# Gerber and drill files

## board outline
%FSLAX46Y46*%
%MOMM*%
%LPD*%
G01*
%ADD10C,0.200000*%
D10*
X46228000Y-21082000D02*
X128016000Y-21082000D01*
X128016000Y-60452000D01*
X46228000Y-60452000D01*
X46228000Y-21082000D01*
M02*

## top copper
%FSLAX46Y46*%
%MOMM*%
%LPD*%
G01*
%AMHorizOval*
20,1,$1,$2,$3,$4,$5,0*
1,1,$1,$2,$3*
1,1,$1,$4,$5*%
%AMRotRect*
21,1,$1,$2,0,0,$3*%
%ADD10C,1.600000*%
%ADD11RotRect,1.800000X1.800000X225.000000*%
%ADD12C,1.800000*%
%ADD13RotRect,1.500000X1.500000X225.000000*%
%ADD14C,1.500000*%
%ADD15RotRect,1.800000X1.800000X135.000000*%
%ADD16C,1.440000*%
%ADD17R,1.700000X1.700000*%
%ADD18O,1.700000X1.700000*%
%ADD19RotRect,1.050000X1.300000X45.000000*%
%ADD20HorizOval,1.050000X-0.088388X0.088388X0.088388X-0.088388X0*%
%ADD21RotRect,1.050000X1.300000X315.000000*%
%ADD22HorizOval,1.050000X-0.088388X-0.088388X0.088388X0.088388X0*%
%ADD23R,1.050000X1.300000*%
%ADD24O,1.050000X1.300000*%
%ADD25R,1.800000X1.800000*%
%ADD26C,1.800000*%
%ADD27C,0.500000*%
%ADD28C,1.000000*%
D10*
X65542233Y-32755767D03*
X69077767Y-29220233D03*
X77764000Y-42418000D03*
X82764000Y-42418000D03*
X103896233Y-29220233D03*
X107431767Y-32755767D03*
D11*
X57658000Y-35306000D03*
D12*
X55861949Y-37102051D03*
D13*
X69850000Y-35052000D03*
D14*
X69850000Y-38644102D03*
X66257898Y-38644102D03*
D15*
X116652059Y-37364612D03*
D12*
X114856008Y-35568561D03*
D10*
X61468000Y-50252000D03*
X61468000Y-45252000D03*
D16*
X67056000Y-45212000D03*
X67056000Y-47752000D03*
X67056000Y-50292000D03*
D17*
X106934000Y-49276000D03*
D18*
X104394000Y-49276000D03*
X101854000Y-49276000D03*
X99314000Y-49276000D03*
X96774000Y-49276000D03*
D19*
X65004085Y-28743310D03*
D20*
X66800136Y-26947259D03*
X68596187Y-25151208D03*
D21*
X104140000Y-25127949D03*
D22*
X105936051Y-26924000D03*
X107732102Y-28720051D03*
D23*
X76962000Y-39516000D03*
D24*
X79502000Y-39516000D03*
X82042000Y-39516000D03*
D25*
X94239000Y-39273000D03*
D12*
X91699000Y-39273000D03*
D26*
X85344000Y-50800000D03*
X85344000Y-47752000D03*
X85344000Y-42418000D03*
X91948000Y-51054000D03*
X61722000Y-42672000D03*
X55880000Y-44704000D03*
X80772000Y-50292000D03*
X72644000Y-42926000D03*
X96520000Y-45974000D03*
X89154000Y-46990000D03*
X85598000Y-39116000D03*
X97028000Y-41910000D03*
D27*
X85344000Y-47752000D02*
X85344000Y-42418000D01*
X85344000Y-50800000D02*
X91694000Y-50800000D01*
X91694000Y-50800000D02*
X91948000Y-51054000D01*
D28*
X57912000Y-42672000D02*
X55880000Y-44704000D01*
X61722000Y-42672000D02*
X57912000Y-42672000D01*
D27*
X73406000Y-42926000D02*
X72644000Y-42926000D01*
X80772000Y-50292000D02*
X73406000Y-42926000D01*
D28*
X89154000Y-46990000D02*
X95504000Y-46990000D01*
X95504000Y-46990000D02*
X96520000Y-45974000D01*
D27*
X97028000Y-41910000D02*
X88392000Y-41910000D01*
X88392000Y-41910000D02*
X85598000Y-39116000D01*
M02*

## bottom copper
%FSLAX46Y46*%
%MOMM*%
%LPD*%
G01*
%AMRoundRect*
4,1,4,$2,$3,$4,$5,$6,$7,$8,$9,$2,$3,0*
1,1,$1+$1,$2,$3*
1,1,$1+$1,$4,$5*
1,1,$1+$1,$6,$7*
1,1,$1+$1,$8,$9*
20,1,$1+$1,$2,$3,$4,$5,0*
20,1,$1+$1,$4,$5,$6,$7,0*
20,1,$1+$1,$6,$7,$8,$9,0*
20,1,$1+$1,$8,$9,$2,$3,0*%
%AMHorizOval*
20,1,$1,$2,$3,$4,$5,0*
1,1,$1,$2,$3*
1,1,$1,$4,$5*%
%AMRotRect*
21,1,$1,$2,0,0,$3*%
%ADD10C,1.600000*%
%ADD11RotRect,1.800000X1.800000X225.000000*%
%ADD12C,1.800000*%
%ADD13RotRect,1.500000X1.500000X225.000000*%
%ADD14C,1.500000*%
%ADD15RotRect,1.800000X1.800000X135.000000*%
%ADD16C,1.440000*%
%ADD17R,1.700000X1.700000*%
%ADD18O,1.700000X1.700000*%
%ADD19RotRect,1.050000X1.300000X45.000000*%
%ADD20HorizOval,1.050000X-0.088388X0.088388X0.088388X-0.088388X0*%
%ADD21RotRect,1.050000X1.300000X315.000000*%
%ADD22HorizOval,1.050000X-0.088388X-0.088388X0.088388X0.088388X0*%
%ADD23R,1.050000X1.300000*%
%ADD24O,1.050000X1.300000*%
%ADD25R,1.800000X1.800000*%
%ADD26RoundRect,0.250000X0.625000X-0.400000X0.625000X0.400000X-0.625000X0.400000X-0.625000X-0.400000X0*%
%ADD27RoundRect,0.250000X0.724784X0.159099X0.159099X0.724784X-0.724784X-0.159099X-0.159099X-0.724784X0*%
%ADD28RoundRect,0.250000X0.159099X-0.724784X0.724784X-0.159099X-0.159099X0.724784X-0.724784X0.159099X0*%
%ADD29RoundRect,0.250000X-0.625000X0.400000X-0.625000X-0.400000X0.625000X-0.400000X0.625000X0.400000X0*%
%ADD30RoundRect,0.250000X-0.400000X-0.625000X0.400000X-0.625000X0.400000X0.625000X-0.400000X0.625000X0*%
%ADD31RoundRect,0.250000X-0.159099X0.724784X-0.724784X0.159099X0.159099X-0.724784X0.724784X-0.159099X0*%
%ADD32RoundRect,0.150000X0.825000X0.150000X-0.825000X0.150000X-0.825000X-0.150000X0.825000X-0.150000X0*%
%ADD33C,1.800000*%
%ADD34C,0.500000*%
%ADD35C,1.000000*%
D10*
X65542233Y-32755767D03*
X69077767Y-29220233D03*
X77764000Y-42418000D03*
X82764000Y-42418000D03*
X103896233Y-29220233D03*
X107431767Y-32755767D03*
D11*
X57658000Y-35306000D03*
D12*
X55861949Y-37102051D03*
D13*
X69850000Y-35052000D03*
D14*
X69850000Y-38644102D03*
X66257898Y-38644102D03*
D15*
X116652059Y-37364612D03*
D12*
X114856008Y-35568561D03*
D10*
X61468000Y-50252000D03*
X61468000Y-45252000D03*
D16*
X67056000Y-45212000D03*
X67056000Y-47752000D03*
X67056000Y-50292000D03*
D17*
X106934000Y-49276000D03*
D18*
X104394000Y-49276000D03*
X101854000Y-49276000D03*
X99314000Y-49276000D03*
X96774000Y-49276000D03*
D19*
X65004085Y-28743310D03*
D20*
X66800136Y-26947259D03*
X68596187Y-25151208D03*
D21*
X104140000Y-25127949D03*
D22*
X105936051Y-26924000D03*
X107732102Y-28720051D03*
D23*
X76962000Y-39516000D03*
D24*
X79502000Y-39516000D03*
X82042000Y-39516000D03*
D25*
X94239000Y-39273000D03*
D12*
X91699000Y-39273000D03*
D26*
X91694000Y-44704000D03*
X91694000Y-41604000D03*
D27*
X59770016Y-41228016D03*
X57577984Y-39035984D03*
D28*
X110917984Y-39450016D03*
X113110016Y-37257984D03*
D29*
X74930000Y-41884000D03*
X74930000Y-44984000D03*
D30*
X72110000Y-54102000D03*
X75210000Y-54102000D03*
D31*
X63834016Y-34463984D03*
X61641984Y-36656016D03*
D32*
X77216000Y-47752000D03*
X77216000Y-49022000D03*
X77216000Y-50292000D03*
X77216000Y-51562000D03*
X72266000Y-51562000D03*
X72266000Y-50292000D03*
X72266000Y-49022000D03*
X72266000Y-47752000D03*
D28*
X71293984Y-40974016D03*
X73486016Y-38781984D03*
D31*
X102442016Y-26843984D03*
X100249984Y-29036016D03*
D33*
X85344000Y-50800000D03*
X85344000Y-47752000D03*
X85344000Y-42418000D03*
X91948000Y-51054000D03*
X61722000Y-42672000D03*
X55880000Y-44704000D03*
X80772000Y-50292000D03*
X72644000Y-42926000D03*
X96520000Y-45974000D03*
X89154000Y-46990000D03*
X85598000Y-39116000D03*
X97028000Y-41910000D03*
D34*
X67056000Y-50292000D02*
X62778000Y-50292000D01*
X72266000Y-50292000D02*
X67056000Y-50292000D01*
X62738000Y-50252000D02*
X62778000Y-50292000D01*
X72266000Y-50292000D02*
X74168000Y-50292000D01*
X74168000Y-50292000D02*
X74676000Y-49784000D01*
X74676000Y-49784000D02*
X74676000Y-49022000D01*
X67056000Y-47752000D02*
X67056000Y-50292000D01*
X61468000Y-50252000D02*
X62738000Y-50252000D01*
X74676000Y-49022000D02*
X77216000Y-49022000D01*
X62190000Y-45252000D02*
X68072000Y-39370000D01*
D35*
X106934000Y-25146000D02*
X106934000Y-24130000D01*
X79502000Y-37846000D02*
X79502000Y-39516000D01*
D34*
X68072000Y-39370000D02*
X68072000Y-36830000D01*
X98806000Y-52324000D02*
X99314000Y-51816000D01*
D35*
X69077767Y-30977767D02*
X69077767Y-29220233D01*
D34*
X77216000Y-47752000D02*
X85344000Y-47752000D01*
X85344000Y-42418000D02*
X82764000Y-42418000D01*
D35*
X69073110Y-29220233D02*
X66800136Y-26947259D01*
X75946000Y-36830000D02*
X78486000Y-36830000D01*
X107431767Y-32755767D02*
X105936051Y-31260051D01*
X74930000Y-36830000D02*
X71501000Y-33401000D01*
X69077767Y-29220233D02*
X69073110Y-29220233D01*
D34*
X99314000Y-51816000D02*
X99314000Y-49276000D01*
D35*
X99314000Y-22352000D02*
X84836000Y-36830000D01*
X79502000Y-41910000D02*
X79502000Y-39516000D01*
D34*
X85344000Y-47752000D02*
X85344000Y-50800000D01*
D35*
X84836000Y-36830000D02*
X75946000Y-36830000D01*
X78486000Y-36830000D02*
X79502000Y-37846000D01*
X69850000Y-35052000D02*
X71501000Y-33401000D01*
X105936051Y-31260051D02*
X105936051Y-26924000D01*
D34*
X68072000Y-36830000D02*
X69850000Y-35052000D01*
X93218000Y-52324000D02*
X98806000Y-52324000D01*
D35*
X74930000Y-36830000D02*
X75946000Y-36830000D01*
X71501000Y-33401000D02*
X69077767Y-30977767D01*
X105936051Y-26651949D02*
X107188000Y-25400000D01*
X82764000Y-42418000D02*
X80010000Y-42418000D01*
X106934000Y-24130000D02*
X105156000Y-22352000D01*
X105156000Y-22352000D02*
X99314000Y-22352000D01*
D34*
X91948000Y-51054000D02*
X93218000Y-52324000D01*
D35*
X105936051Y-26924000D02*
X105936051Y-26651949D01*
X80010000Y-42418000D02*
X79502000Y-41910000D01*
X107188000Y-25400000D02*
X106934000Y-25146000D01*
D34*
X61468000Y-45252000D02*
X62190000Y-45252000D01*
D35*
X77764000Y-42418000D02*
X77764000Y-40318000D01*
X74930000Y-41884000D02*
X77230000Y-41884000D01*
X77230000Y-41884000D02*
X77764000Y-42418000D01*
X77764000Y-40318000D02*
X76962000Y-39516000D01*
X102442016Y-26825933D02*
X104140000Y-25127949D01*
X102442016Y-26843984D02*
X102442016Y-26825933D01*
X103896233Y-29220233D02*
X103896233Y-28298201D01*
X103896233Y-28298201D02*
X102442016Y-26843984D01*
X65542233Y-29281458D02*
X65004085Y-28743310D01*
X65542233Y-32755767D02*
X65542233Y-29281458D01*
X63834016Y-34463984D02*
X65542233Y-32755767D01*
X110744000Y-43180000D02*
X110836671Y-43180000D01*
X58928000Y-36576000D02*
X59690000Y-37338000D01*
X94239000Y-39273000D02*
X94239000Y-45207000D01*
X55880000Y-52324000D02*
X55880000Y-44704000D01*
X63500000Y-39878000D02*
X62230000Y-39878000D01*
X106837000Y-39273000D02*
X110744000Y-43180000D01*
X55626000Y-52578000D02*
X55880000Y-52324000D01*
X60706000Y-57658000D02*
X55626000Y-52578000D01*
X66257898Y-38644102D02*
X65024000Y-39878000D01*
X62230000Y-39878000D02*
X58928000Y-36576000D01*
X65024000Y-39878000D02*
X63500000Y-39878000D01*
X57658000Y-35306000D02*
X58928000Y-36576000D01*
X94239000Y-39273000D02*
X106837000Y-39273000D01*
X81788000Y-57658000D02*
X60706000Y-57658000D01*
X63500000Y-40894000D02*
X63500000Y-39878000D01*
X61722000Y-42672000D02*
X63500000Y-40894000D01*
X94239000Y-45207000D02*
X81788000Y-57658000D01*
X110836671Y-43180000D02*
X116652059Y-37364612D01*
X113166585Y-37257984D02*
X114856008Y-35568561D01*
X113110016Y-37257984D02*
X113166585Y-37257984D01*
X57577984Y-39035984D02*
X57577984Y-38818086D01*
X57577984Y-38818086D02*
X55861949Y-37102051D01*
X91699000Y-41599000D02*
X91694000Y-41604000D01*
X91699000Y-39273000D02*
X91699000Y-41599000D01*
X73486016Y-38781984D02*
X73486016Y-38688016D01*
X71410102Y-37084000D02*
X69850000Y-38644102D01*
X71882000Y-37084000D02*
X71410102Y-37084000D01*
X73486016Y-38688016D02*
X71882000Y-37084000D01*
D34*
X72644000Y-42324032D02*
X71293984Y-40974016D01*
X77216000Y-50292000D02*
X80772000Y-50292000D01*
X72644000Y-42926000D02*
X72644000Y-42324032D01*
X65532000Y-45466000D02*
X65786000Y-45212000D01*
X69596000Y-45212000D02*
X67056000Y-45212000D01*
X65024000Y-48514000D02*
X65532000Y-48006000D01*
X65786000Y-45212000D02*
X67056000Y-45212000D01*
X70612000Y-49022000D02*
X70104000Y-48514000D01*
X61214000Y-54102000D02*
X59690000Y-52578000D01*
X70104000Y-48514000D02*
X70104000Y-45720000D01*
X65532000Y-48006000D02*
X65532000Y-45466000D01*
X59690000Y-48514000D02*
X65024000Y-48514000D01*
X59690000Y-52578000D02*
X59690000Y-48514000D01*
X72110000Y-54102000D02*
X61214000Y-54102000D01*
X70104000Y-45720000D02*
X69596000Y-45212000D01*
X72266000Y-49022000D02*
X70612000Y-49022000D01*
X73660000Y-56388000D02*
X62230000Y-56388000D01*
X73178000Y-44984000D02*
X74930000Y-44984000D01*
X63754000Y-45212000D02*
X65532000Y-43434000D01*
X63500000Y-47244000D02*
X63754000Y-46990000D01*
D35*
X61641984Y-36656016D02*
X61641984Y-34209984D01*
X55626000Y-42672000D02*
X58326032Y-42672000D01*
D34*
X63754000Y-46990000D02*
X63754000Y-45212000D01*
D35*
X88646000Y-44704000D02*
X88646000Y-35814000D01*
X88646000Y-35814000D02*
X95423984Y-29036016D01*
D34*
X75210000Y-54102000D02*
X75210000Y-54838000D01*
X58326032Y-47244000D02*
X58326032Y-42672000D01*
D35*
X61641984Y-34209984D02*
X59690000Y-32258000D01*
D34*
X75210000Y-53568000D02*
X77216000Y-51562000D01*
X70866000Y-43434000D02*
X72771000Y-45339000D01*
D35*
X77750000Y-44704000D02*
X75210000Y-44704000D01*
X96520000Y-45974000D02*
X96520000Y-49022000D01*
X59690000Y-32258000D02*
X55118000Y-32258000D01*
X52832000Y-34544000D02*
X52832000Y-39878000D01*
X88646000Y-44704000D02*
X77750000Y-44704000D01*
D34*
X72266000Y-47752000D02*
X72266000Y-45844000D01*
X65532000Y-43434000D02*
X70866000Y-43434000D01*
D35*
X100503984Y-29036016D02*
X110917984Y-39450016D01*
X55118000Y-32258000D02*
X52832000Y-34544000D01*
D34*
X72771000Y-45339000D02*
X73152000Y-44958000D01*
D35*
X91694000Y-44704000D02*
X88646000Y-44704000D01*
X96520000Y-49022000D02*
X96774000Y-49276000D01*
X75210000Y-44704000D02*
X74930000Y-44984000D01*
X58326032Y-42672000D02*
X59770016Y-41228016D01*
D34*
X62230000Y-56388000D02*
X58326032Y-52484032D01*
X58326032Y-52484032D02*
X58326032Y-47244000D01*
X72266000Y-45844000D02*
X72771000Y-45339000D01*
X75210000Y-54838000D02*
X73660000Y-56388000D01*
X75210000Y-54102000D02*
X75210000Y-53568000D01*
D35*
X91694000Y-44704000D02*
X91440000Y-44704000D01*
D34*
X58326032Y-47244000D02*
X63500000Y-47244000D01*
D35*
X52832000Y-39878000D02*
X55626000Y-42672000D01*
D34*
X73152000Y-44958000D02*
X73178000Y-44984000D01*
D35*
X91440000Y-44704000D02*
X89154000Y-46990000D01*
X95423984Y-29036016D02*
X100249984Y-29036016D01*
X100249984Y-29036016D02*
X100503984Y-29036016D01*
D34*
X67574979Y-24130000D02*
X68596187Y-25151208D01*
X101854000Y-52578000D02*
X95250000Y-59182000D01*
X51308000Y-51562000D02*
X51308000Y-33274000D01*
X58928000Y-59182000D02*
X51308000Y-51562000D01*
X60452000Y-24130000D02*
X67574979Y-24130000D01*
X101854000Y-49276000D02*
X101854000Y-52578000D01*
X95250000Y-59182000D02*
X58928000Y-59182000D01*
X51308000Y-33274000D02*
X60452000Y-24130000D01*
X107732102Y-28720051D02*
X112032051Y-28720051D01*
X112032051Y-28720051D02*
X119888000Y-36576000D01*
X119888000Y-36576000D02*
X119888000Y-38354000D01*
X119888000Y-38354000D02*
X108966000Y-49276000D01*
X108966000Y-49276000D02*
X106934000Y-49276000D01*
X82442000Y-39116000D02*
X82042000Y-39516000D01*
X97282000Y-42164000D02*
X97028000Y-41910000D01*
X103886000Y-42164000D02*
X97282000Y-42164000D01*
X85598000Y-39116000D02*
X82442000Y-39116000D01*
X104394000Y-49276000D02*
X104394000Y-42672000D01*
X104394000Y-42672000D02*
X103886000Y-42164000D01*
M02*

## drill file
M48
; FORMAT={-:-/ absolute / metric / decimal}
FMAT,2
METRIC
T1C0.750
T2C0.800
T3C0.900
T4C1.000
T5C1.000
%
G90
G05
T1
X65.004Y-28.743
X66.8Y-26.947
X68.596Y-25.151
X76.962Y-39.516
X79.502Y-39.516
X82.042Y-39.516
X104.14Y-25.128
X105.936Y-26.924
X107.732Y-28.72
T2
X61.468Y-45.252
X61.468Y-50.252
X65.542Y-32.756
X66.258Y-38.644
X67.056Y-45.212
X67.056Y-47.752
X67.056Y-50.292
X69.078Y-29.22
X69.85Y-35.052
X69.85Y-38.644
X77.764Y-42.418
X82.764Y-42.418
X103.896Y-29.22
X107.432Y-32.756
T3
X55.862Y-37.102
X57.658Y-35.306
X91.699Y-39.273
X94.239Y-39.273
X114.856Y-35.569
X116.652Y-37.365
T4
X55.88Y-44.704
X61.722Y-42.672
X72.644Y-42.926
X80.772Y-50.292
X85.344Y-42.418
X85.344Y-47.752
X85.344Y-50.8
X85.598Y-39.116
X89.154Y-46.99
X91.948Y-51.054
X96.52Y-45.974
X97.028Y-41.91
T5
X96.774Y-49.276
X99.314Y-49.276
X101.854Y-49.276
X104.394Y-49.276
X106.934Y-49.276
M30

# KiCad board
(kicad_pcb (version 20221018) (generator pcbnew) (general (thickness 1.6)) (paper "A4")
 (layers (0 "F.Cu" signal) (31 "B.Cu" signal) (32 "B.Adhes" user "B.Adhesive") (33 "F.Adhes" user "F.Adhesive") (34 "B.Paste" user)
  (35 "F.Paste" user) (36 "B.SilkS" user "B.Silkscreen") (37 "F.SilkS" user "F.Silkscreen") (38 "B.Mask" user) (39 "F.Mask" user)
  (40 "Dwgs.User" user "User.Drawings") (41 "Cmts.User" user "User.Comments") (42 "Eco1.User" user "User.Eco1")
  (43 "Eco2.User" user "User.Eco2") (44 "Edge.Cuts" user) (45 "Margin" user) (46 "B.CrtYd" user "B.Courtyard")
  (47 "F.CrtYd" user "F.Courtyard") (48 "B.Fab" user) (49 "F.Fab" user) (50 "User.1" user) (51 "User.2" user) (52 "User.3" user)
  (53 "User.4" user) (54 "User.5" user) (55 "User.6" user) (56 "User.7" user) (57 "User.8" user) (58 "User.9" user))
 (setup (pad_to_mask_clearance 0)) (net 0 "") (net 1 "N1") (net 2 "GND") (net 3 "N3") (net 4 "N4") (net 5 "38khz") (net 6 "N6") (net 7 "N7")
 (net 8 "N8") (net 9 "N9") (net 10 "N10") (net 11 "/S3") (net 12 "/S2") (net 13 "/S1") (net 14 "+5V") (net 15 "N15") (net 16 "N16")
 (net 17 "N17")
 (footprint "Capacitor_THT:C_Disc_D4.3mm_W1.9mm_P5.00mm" (layer "F.Cu") (at 65.542233 32.755767 45)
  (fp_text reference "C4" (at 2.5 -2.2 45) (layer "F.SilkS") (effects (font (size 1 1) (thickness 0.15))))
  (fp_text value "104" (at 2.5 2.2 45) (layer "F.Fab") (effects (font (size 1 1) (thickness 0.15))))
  (pad "1" thru_hole circle (at 0 0 45) (size 1.6 1.6) (drill 0.8) (layers "*.Cu" "*.Mask") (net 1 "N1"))
  (pad "2" thru_hole circle (at 5 0 45) (size 1.6 1.6) (drill 0.8) (layers "*.Cu" "*.Mask") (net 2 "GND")))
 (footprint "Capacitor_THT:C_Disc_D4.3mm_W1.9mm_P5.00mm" (layer "F.Cu") (at 77.764 42.418)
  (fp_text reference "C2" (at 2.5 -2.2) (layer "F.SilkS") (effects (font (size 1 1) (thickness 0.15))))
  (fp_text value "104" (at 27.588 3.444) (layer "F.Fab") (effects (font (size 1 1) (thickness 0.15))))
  (pad "1" thru_hole circle (at 0 0) (size 1.6 1.6) (drill 0.8) (layers "*.Cu" "*.Mask") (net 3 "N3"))
  (pad "2" thru_hole circle (at 5 0) (size 1.6 1.6) (drill 0.8) (layers "*.Cu" "*.Mask") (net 2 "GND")))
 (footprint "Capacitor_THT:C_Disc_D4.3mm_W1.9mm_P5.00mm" (layer "F.Cu") (at 103.896233 29.220233 -45)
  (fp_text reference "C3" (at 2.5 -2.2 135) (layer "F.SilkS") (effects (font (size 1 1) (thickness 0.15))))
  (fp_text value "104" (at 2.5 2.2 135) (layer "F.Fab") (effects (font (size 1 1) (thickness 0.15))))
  (pad "1" thru_hole circle (at 0 0 315) (size 1.6 1.6) (drill 0.8) (layers "*.Cu" "*.Mask") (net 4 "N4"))
  (pad "2" thru_hole circle (at 5 0 315) (size 1.6 1.6) (drill 0.8) (layers "*.Cu" "*.Mask") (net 2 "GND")))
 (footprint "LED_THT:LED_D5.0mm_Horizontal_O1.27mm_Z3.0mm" (layer "F.Cu") (at 57.658 35.306 -135)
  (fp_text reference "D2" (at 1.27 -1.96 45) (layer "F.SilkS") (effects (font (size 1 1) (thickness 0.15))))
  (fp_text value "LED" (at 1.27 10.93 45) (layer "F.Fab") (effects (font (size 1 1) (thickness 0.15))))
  (pad "1" thru_hole rect (at 0 0 225) (size 1.8 1.8) (drill 0.9) (layers "*.Cu" "*.Mask") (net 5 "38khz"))
  (pad "2" thru_hole circle (at 2.54 0 225) (size 1.8 1.8) (drill 0.9) (layers "*.Cu" "*.Mask") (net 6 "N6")))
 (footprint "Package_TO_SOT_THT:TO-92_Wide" (layer "F.Cu") (at 69.85 35.052 -135)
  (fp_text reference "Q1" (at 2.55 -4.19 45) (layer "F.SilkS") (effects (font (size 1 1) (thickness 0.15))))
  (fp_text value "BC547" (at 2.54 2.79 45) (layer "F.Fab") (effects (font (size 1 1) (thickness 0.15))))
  (pad "1" thru_hole rect (at 0 0 225) (size 1.5 1.5) (drill 0.8) (layers "*.Cu" "*.Mask") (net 2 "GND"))
  (pad "2" thru_hole circle (at 2.54 -2.54 225) (size 1.5 1.5) (drill 0.8) (layers "*.Cu" "*.Mask") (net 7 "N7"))
  (pad "3" thru_hole circle (at 5.08 0 225) (size 1.5 1.5) (drill 0.8) (layers "*.Cu" "*.Mask") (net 5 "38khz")))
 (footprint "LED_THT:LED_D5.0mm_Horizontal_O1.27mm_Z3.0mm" (layer "F.Cu") (at 116.652059 37.364612 135)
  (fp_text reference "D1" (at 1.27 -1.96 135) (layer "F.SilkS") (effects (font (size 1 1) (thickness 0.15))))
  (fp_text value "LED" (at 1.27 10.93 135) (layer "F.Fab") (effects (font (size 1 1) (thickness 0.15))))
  (pad "1" thru_hole rect (at 0 0 135) (size 1.8 1.8) (drill 0.9) (layers "*.Cu" "*.Mask") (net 5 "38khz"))
  (pad "2" thru_hole circle (at 2.54 0 135) (size 1.8 1.8) (drill 0.9) (layers "*.Cu" "*.Mask") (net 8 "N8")))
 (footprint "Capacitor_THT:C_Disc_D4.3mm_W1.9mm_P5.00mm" (layer "F.Cu") (at 61.468 50.252 90)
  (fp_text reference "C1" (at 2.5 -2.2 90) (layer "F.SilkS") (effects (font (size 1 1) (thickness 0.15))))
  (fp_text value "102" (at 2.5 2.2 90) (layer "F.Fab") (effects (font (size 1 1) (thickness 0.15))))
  (pad "1" thru_hole circle (at 0 0 90) (size 1.6 1.6) (drill 0.8) (layers "*.Cu" "*.Mask") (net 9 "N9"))
  (pad "2" thru_hole circle (at 5 0 90) (size 1.6 1.6) (drill 0.8) (layers "*.Cu" "*.Mask") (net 2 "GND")))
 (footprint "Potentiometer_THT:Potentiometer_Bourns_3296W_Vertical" (layer "F.Cu") (at 67.056 45.212 90)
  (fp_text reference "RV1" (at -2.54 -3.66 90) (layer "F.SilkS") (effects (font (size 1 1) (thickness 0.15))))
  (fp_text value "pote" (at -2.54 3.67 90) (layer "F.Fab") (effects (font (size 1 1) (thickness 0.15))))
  (pad "1" thru_hole circle (at 0 0 90) (size 1.44 1.44) (drill 0.8) (layers "*.Cu" "*.Mask") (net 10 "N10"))
  (pad "2" thru_hole circle (at -2.54 0 90) (size 1.44 1.44) (drill 0.8) (layers "*.Cu" "*.Mask") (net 9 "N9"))
  (pad "3" thru_hole circle (at -5.08 0 90) (size 1.44 1.44) (drill 0.8) (layers "*.Cu" "*.Mask") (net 9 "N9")))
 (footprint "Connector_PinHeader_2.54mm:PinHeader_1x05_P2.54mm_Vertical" (layer "F.Cu") (at 106.934 49.276 -90)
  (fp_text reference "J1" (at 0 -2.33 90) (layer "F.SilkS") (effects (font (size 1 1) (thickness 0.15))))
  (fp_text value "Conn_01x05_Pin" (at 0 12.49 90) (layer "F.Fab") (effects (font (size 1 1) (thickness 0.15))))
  (pad "1" thru_hole rect (at 0 0 270) (size 1.7 1.7) (drill 1) (layers "*.Cu" "*.Mask") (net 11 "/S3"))
  (pad "2" thru_hole oval (at 0 2.54 270) (size 1.7 1.7) (drill 1) (layers "*.Cu" "*.Mask") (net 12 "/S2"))
  (pad "3" thru_hole oval (at 0 5.08 270) (size 1.7 1.7) (drill 1) (layers "*.Cu" "*.Mask") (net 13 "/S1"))
  (pad "4" thru_hole oval (at 0 7.62 270) (size 1.7 1.7) (drill 1) (layers "*.Cu" "*.Mask") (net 2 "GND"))
  (pad "5" thru_hole oval (at 0 10.16 270) (size 1.7 1.7) (drill 1) (layers "*.Cu" "*.Mask") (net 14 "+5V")))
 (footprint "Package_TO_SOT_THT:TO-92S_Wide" (layer "F.Cu") (at 65.004085 28.74331 45)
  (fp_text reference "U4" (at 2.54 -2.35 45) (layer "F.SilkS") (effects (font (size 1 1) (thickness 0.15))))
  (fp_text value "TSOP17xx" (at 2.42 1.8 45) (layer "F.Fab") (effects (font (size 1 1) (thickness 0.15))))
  (pad "1" thru_hole rect (at 0 0 45) (size 1.05 1.3) (drill 0.75) (layers "*.Cu" "*.Mask") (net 1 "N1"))
  (pad "2" thru_hole oval (at 2.54 0 45) (size 1.05 1.3) (drill 0.75) (layers "*.Cu" "*.Mask") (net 2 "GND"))
  (pad "3" thru_hole oval (at 5.08 0 45) (size 1.05 1.3) (drill 0.75) (layers "*.Cu" "*.Mask") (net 13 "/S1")))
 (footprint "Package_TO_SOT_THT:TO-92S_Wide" (layer "F.Cu") (at 104.14 25.127949 -45)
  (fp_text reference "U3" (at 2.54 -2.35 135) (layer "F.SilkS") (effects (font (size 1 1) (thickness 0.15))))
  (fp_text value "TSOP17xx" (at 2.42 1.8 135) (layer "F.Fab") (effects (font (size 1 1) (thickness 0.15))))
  (pad "1" thru_hole rect (at 0 0 315) (size 1.05 1.3) (drill 0.75) (layers "*.Cu" "*.Mask") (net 4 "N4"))
  (pad "2" thru_hole oval (at 2.54 0 315) (size 1.05 1.3) (drill 0.75) (layers "*.Cu" "*.Mask") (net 2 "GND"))
  (pad "3" thru_hole oval (at 5.08 0 315) (size 1.05 1.3) (drill 0.75) (layers "*.Cu" "*.Mask") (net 11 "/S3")))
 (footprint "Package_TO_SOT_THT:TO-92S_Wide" (layer "F.Cu") (at 76.962 39.516)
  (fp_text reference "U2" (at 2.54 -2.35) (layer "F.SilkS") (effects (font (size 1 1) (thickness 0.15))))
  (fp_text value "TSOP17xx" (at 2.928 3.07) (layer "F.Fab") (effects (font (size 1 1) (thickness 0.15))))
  (pad "1" thru_hole rect (at 0 0) (size 1.05 1.3) (drill 0.75) (layers "*.Cu" "*.Mask") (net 3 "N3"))
  (pad "2" thru_hole oval (at 2.54 0) (size 1.05 1.3) (drill 0.75) (layers "*.Cu" "*.Mask") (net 2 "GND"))
  (pad "3" thru_hole oval (at 5.08 0) (size 1.05 1.3) (drill 0.75) (layers "*.Cu" "*.Mask") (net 12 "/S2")))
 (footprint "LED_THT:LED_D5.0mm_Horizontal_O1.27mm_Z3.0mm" (layer "F.Cu") (at 94.239 39.273 180)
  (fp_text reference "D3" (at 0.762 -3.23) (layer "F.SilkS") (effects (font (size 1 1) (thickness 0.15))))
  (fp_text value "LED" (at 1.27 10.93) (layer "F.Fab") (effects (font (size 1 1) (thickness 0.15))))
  (pad "1" thru_hole rect (at 0 0 180) (size 1.8 1.8) (drill 0.9) (layers "*.Cu" "*.Mask") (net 5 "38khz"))
  (pad "2" thru_hole circle (at 2.54 0 180) (size 1.8 1.8) (drill 0.9) (layers "*.Cu" "*.Mask") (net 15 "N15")))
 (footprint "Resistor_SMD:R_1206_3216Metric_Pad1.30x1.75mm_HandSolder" (layer "B.Cu") (at 91.694 43.154 90)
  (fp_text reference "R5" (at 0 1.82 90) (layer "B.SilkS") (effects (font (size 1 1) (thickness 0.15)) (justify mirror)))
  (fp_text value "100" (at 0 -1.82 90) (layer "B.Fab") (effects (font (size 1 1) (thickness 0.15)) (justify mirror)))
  (pad "1" smd roundrect (at -1.55 0 90) (size 1.3 1.75) (layers "B.Cu" "B.Paste" "B.Mask") (roundrect_rratio 0.192308) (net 14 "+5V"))
  (pad "2" smd roundrect (at 1.55 0 90) (size 1.3 1.75) (layers "B.Cu" "B.Paste" "B.Mask") (roundrect_rratio 0.192308) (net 15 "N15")))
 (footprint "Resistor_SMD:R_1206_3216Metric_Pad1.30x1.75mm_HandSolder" (layer "B.Cu") (at 58.674 40.132 135)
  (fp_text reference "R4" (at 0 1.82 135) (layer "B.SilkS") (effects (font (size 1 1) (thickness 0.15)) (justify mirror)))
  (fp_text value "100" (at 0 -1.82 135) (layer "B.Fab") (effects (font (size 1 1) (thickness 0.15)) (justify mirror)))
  (pad "1" smd roundrect (at -1.55 0 135) (size 1.3 1.75) (layers "B.Cu" "B.Paste" "B.Mask") (roundrect_rratio 0.192308) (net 14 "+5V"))
  (pad "2" smd roundrect (at 1.55 0 135) (size 1.3 1.75) (layers "B.Cu" "B.Paste" "B.Mask") (roundrect_rratio 0.192308) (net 6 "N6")))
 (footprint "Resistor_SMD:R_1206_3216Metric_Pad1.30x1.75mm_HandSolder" (layer "B.Cu") (at 112.014 38.354 45)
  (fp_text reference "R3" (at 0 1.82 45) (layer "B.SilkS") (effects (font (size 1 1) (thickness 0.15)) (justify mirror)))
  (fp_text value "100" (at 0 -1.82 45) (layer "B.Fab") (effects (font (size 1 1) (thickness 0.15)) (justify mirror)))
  (pad "1" smd roundrect (at -1.55 0 45) (size 1.3 1.75) (layers "B.Cu" "B.Paste" "B.Mask") (roundrect_rratio 0.192308) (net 14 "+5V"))
  (pad "2" smd roundrect (at 1.55 0 45) (size 1.3 1.75) (layers "B.Cu" "B.Paste" "B.Mask") (roundrect_rratio 0.192308) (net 8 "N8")))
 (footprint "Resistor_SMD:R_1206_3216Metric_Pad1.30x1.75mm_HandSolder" (layer "B.Cu") (at 74.93 43.434 -90)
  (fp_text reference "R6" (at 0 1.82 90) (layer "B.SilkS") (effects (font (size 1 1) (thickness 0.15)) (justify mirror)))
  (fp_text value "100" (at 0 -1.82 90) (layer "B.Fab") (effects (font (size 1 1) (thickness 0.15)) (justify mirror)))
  (pad "1" smd roundrect (at -1.55 0 270) (size 1.3 1.75) (layers "B.Cu" "B.Paste" "B.Mask") (roundrect_rratio 0.192308) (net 3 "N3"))
  (pad "2" smd roundrect (at 1.55 0 270) (size 1.3 1.75) (layers "B.Cu" "B.Paste" "B.Mask") (roundrect_rratio 0.192308) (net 14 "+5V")))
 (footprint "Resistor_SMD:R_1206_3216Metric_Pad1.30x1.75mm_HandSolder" (layer "B.Cu") (at 73.66 54.102)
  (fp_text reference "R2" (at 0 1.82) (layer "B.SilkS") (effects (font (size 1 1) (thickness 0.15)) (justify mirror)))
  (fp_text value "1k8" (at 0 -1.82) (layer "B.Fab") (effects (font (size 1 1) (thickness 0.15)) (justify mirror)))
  (pad "1" smd roundrect (at -1.55 0) (size 1.3 1.75) (layers "B.Cu" "B.Paste" "B.Mask") (roundrect_rratio 0.192308) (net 10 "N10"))
  (pad "2" smd roundrect (at 1.55 0) (size 1.3 1.75) (layers "B.Cu" "B.Paste" "B.Mask") (roundrect_rratio 0.192308) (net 14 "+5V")))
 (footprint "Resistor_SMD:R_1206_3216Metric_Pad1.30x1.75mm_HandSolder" (layer "B.Cu") (at 62.738 35.56 -135)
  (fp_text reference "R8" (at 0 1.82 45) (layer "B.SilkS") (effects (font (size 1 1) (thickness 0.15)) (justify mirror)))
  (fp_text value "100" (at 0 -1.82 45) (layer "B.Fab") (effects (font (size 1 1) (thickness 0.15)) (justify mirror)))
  (pad "1" smd roundrect (at -1.55 0 225) (size 1.3 1.75) (layers "B.Cu" "B.Paste" "B.Mask") (roundrect_rratio 0.192308) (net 1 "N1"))
  (pad "2" smd roundrect (at 1.55 0 225) (size 1.3 1.75) (layers "B.Cu" "B.Paste" "B.Mask") (roundrect_rratio 0.192308) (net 14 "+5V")))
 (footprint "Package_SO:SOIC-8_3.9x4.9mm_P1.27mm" (layer "B.Cu") (at 74.741 49.657 180)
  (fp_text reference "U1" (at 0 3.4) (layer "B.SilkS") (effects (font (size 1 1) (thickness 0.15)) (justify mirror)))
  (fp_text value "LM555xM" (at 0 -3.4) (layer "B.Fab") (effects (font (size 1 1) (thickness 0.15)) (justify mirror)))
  (pad "1" smd roundrect (at -2.475 1.905 180) (size 1.95 0.6) (layers "B.Cu" "B.Paste" "B.Mask") (roundrect_rratio 0.25) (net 2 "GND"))
  (pad "2" smd roundrect (at -2.475 0.635 180) (size 1.95 0.6) (layers "B.Cu" "B.Paste" "B.Mask") (roundrect_rratio 0.25) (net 9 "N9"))
  (pad "3" smd roundrect (at -2.475 -0.635 180) (size 1.95 0.6) (layers "B.Cu" "B.Paste" "B.Mask") (roundrect_rratio 0.25) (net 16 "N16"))
  (pad "4" smd roundrect (at -2.475 -1.905 180) (size 1.95 0.6) (layers "B.Cu" "B.Paste" "B.Mask") (roundrect_rratio 0.25) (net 14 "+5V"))
  (pad "5" smd roundrect (at 2.475 -1.905 180) (size 1.95 0.6) (layers "B.Cu" "B.Paste" "B.Mask") (roundrect_rratio 0.25) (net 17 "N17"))
  (pad "6" smd roundrect (at 2.475 -0.635 180) (size 1.95 0.6) (layers "B.Cu" "B.Paste" "B.Mask") (roundrect_rratio 0.25) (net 9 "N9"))
  (pad "7" smd roundrect (at 2.475 0.635 180) (size 1.95 0.6) (layers "B.Cu" "B.Paste" "B.Mask") (roundrect_rratio 0.25) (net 10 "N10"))
  (pad "8" smd roundrect (at 2.475 1.905 180) (size 1.95 0.6) (layers "B.Cu" "B.Paste" "B.Mask") (roundrect_rratio 0.25) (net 14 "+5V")))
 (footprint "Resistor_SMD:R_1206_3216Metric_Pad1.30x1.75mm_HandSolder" (layer "B.Cu") (at 72.39 39.878 45)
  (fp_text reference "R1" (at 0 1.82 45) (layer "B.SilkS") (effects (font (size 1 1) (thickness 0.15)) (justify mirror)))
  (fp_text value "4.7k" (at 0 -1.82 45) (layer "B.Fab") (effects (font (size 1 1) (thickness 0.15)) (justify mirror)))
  (pad "1" smd roundrect (at -1.55 0 45) (size 1.3 1.75) (layers "B.Cu" "B.Paste" "B.Mask") (roundrect_rratio 0.192308) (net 16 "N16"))
  (pad "2" smd roundrect (at 1.55 0 45) (size 1.3 1.75) (layers "B.Cu" "B.Paste" "B.Mask") (roundrect_rratio 0.192308) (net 7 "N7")))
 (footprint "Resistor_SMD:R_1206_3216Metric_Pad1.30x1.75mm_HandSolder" (layer "B.Cu") (at 101.346 27.94 -135)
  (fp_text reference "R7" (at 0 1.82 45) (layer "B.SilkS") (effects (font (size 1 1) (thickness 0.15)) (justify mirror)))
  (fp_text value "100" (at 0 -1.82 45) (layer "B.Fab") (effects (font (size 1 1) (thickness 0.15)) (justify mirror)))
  (pad "1" smd roundrect (at -1.55 0 225) (size 1.3 1.75) (layers "B.Cu" "B.Paste" "B.Mask") (roundrect_rratio 0.192308) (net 4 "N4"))
  (pad "2" smd roundrect (at 1.55 0 225) (size 1.3 1.75) (layers "B.Cu" "B.Paste" "B.Mask") (roundrect_rratio 0.192308) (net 14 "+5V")))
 (gr_rect (start 46.228 21.082) (end 128.016 60.452) (stroke (width 0.2) (type default)) (fill none) (layer "Edge.Cuts"))
 (segment (start 67.056 50.292) (end 62.778 50.292) (width 0.5) (layer "B.Cu") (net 9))
 (segment (start 72.266 50.292) (end 67.056 50.292) (width 0.5) (layer "B.Cu") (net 9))
 (segment (start 62.738 50.252) (end 62.778 50.292) (width 0.5) (layer "B.Cu") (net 9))
 (segment (start 72.266 50.292) (end 74.168 50.292) (width 0.5) (layer "B.Cu") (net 9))
 (segment (start 74.168 50.292) (end 74.676 49.784) (width 0.5) (layer "B.Cu") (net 9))
 (segment (start 74.676 49.784) (end 74.676 49.022) (width 0.5) (layer "B.Cu") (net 9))
 (segment (start 67.056 47.752) (end 67.056 50.292) (width 0.5) (layer "B.Cu") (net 9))
 (segment (start 61.468 50.252) (end 62.738 50.252) (width 0.5) (layer "B.Cu") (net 9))
 (segment (start 74.676 49.022) (end 77.216 49.022) (width 0.5) (layer "B.Cu") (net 9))
 (segment (start 85.344 47.752) (end 85.344 42.418) (width 0.5) (layer "F.Cu") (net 2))
 (segment (start 85.344 50.8) (end 91.694 50.8) (width 0.5) (layer "F.Cu") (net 2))
 (segment (start 91.694 50.8) (end 91.948 51.054) (width 0.5) (layer "F.Cu") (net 2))
 (via (at 85.344 50.8) (size 1.8) (drill 1) (layers "F.Cu" "B.Cu") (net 2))
 (via (at 85.344 47.752) (size 1.8) (drill 1) (layers "F.Cu" "B.Cu") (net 2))
 (via (at 85.344 42.418) (size 1.8) (drill 1) (layers "F.Cu" "B.Cu") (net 2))
 (via (at 91.948 51.054) (size 1.8) (drill 1) (layers "F.Cu" "B.Cu") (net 2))
 (segment (start 62.19 45.252) (end 68.072 39.37) (width 0.5) (layer "B.Cu") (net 2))
 (segment (start 106.934 25.146) (end 106.934 24.13) (width 1) (layer "B.Cu") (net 2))
 (segment (start 79.502 37.846) (end 79.502 39.516) (width 1) (layer "B.Cu") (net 2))
 (segment (start 68.072 39.37) (end 68.072 36.83) (width 0.5) (layer "B.Cu") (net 2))
 (segment (start 98.806 52.324) (end 99.314 51.816) (width 0.5) (layer "B.Cu") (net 2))
 (segment (start 69.077767 30.977767) (end 69.077767 29.220233) (width 1) (layer "B.Cu") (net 2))
 (segment (start 77.216 47.752) (end 85.344 47.752) (width 0.5) (layer "B.Cu") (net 2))
 (segment (start 85.344 42.418) (end 82.764 42.418) (width 0.5) (layer "B.Cu") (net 2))
 (segment (start 69.07311 29.220233) (end 66.800136 26.947259) (width 1) (layer "B.Cu") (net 2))
 (segment (start 75.946 36.83) (end 78.486 36.83) (width 1) (layer "B.Cu") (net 2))
 (segment (start 107.431767 32.755767) (end 105.936051 31.260051) (width 1) (layer "B.Cu") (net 2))
 (segment (start 74.93 36.83) (end 71.501 33.401) (width 1) (layer "B.Cu") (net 2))
 (segment (start 69.077767 29.220233) (end 69.07311 29.220233) (width 1) (layer "B.Cu") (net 2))
 (segment (start 99.314 51.816) (end 99.314 49.276) (width 0.5) (layer "B.Cu") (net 2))
 (segment (start 99.314 22.352) (end 84.836 36.83) (width 1) (layer "B.Cu") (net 2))
 (segment (start 79.502 41.91) (end 79.502 39.516) (width 1) (layer "B.Cu") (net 2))
 (segment (start 85.344 47.752) (end 85.344 50.8) (width 0.5) (layer "B.Cu") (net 2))
 (segment (start 84.836 36.83) (end 75.946 36.83) (width 1) (layer "B.Cu") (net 2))
 (segment (start 78.486 36.83) (end 79.502 37.846) (width 1) (layer "B.Cu") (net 2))
 (segment (start 69.85 35.052) (end 71.501 33.401) (width 1) (layer "B.Cu") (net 2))
 (segment (start 105.936051 31.260051) (end 105.936051 26.924) (width 1) (layer "B.Cu") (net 2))
 (segment (start 68.072 36.83) (end 69.85 35.052) (width 0.5) (layer "B.Cu") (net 2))
 (segment (start 93.218 52.324) (end 98.806 52.324) (width 0.5) (layer "B.Cu") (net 2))
 (segment (start 74.93 36.83) (end 75.946 36.83) (width 1) (layer "B.Cu") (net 2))
 (segment (start 71.501 33.401) (end 69.077767 30.977767) (width 1) (layer "B.Cu") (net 2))
 (segment (start 105.936051 26.651949) (end 107.188 25.4) (width 1) (layer "B.Cu") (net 2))
 (segment (start 82.764 42.418) (end 80.01 42.418) (width 1) (layer "B.Cu") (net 2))
 (segment (start 106.934 24.13) (end 105.156 22.352) (width 1) (layer "B.Cu") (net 2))
 (segment (start 105.156 22.352) (end 99.314 22.352) (width 1) (layer "B.Cu") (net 2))
 (segment (start 91.948 51.054) (end 93.218 52.324) (width 0.5) (layer "B.Cu") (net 2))
 (segment (start 105.936051 26.924) (end 105.936051 26.651949) (width 1) (layer "B.Cu") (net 2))
 (segment (start 80.01 42.418) (end 79.502 41.91) (width 1) (layer "B.Cu") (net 2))
 (segment (start 107.188 25.4) (end 106.934 25.146) (width 1) (layer "B.Cu") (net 2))
 (segment (start 61.468 45.252) (end 62.19 45.252) (width 0.5) (layer "B.Cu") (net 2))
 (segment (start 77.764 42.418) (end 77.764 40.318) (width 1) (layer "B.Cu") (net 3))
 (segment (start 74.93 41.884) (end 77.23 41.884) (width 1) (layer "B.Cu") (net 3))
 (segment (start 77.23 41.884) (end 77.764 42.418) (width 1) (layer "B.Cu") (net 3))
 (segment (start 77.764 40.318) (end 76.962 39.516) (width 1) (layer "B.Cu") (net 3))
 (segment (start 102.442016 26.825933) (end 104.14 25.127949) (width 1) (layer "B.Cu") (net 4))
 (segment (start 102.442016 26.843984) (end 102.442016 26.825933) (width 1) (layer "B.Cu") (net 4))
 (segment (start 103.896233 29.220233) (end 103.896233 28.298201) (width 1) (layer "B.Cu") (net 4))
 (segment (start 103.896233 28.298201) (end 102.442016 26.843984) (width 1) (layer "B.Cu") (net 4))
 (segment (start 65.542233 29.281458) (end 65.004085 28.74331) (width 1) (layer "B.Cu") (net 1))
 (segment (start 65.542233 32.755767) (end 65.542233 29.281458) (width 1) (layer "B.Cu") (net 1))
 (segment (start 63.834016 34.463984) (end 65.542233 32.755767) (width 1) (layer "B.Cu") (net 1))
 (segment (start 57.912 42.672) (end 55.88 44.704) (width 1) (layer "F.Cu") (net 5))
 (segment (start 61.722 42.672) (end 57.912 42.672) (width 1) (layer "F.Cu") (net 5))
 (via (at 61.722 42.672) (size 1.8) (drill 1) (layers "F.Cu" "B.Cu") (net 5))
 (via (at 55.88 44.704) (size 1.8) (drill 1) (layers "F.Cu" "B.Cu") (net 5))
 (segment (start 110.744 43.18) (end 110.836671 43.18) (width 1) (layer "B.Cu") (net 5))
 (segment (start 58.928 36.576) (end 59.69 37.338) (width 1) (layer "B.Cu") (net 5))
 (segment (start 94.239 39.273) (end 94.239 45.207) (width 1) (layer "B.Cu") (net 5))
 (segment (start 55.88 52.324) (end 55.88 44.704) (width 1) (layer "B.Cu") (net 5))
 (segment (start 63.5 39.878) (end 62.23 39.878) (width 1) (layer "B.Cu") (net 5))
 (segment (start 106.837 39.273) (end 110.744 43.18) (width 1) (layer "B.Cu") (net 5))
 (segment (start 55.626 52.578) (end 55.88 52.324) (width 1) (layer "B.Cu") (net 5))
 (segment (start 60.706 57.658) (end 55.626 52.578) (width 1) (layer "B.Cu") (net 5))
 (segment (start 66.257898 38.644102) (end 65.024 39.878) (width 1) (layer "B.Cu") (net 5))
 (segment (start 62.23 39.878) (end 58.928 36.576) (width 1) (layer "B.Cu") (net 5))
 (segment (start 65.024 39.878) (end 63.5 39.878) (width 1) (layer "B.Cu") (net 5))
 (segment (start 57.658 35.306) (end 58.928 36.576) (width 1) (layer "B.Cu") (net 5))
 (segment (start 94.239 39.273) (end 106.837 39.273) (width 1) (layer "B.Cu") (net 5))
 (segment (start 81.788 57.658) (end 60.706 57.658) (width 1) (layer "B.Cu") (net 5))
 (segment (start 63.5 40.894) (end 63.5 39.878) (width 1) (layer "B.Cu") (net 5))
 (segment (start 61.722 42.672) (end 63.5 40.894) (width 1) (layer "B.Cu") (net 5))
 (segment (start 94.239 45.207) (end 81.788 57.658) (width 1) (layer "B.Cu") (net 5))
 (segment (start 110.836671 43.18) (end 116.652059 37.364612) (width 1) (layer "B.Cu") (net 5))
 (segment (start 113.166585 37.257984) (end 114.856008 35.568561) (width 1) (layer "B.Cu") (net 8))
 (segment (start 113.110016 37.257984) (end 113.166585 37.257984) (width 1) (layer "B.Cu") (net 8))
 (segment (start 57.577984 39.035984) (end 57.577984 38.818086) (width 1) (layer "B.Cu") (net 6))
 (segment (start 57.577984 38.818086) (end 55.861949 37.102051) (width 1) (layer "B.Cu") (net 6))
 (segment (start 91.699 41.599) (end 91.694 41.604) (width 1) (layer "B.Cu") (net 15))
 (segment (start 91.699 39.273) (end 91.699 41.599) (width 1) (layer "B.Cu") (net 15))
 (segment (start 73.486016 38.781984) (end 73.486016 38.688016) (width 1) (layer "B.Cu") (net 7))
 (segment (start 71.410102 37.084) (end 69.85 38.644102) (width 1) (layer "B.Cu") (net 7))
 (segment (start 71.882 37.084) (end 71.410102 37.084) (width 1) (layer "B.Cu") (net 7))
 (segment (start 73.486016 38.688016) (end 71.882 37.084) (width 1) (layer "B.Cu") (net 7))
 (segment (start 73.406 42.926) (end 72.644 42.926) (width 0.5) (layer "F.Cu") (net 16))
 (segment (start 80.772 50.292) (end 73.406 42.926) (width 0.5) (layer "F.Cu") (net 16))
 (via (at 80.772 50.292) (size 1.8) (drill 1) (layers "F.Cu" "B.Cu") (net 16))
 (via (at 72.644 42.926) (size 1.8) (drill 1) (layers "F.Cu" "B.Cu") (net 16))
 (segment (start 72.644 42.324032) (end 71.293984 40.974016) (width 0.5) (layer "B.Cu") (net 16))
 (segment (start 77.216 50.292) (end 80.772 50.292) (width 0.5) (layer "B.Cu") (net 16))
 (segment (start 72.644 42.926) (end 72.644 42.324032) (width 0.5) (layer "B.Cu") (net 16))
 (segment (start 65.532 45.466) (end 65.786 45.212) (width 0.5) (layer "B.Cu") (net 10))
 (segment (start 69.596 45.212) (end 67.056 45.212) (width 0.5) (layer "B.Cu") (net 10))
 (segment (start 65.024 48.514) (end 65.532 48.006) (width 0.5) (layer "B.Cu") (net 10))
 (segment (start 65.786 45.212) (end 67.056 45.212) (width 0.5) (layer "B.Cu") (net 10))
 (segment (start 70.612 49.022) (end 70.104 48.514) (width 0.5) (layer "B.Cu") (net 10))
 (segment (start 61.214 54.102) (end 59.69 52.578) (width 0.5) (layer "B.Cu") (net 10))
 (segment (start 70.104 48.514) (end 70.104 45.72) (width 0.5) (layer "B.Cu") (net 10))
 (segment (start 65.532 48.006) (end 65.532 45.466) (width 0.5) (layer "B.Cu") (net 10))
 (segment (start 59.69 48.514) (end 65.024 48.514) (width 0.5) (layer "B.Cu") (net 10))
 (segment (start 59.69 52.578) (end 59.69 48.514) (width 0.5) (layer "B.Cu") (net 10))
 (segment (start 72.11 54.102) (end 61.214 54.102) (width 0.5) (layer "B.Cu") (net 10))
 (segment (start 70.104 45.72) (end 69.596 45.212) (width 0.5) (layer "B.Cu") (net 10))
 (segment (start 72.266 49.022) (end 70.612 49.022) (width 0.5) (layer "B.Cu") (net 10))
 (segment (start 89.154 46.99) (end 95.504 46.99) (width 1) (layer "F.Cu") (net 14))
 (segment (start 95.504 46.99) (end 96.52 45.974) (width 1) (layer "F.Cu") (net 14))
 (via (at 96.52 45.974) (size 1.8) (drill 1) (layers "F.Cu" "B.Cu") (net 14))
 (via (at 89.154 46.99) (size 1.8) (drill 1) (layers "F.Cu" "B.Cu") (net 14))
 (segment (start 73.66 56.388) (end 62.23 56.388) (width 0.5) (layer "B.Cu") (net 14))
 (segment (start 73.178 44.984) (end 74.93 44.984) (width 0.5) (layer "B.Cu") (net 14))
 (segment (start 63.754 45.212) (end 65.532 43.434) (width 0.5) (layer "B.Cu") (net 14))
 (segment (start 63.5 47.244) (end 63.754 46.99) (width 0.5) (layer "B.Cu") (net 14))
 (segment (start 61.641984 36.656016) (end 61.641984 34.209984) (width 1) (layer "B.Cu") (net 14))
 (segment (start 55.626 42.672) (end 58.326032 42.672) (width 1) (layer "B.Cu") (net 14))
 (segment (start 63.754 46.99) (end 63.754 45.212) (width 0.5) (layer "B.Cu") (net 14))
 (segment (start 88.646 44.704) (end 88.646 35.814) (width 1) (layer "B.Cu") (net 14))
 (segment (start 88.646 35.814) (end 95.423984 29.036016) (width 1) (layer "B.Cu") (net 14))
 (segment (start 75.21 54.102) (end 75.21 54.838) (width 0.5) (layer "B.Cu") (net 14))
 (segment (start 58.326032 47.244) (end 58.326032 42.672) (width 0.5) (layer "B.Cu") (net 14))
 (segment (start 61.641984 34.209984) (end 59.69 32.258) (width 1) (layer "B.Cu") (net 14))
 (segment (start 75.21 53.568) (end 77.216 51.562) (width 0.5) (layer "B.Cu") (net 14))
 (segment (start 70.866 43.434) (end 72.771 45.339) (width 0.5) (layer "B.Cu") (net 14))
 (segment (start 77.75 44.704) (end 75.21 44.704) (width 1) (layer "B.Cu") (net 14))
 (segment (start 96.52 45.974) (end 96.52 49.022) (width 1) (layer "B.Cu") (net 14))
 (segment (start 59.69 32.258) (end 55.118 32.258) (width 1) (layer "B.Cu") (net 14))
 (segment (start 52.832 34.544) (end 52.832 39.878) (width 1) (layer "B.Cu") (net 14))
 (segment (start 88.646 44.704) (end 77.75 44.704) (width 1) (layer "B.Cu") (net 14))
 (segment (start 72.266 47.752) (end 72.266 45.844) (width 0.5) (layer "B.Cu") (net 14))
 (segment (start 65.532 43.434) (end 70.866 43.434) (width 0.5) (layer "B.Cu") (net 14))
 (segment (start 100.503984 29.036016) (end 110.917984 39.450016) (width 1) (layer "B.Cu") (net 14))
 (segment (start 55.118 32.258) (end 52.832 34.544) (width 1) (layer "B.Cu") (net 14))
 (segment (start 72.771 45.339) (end 73.152 44.958) (width 0.5) (layer "B.Cu") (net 14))
 (segment (start 91.694 44.704) (end 88.646 44.704) (width 1) (layer "B.Cu") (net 14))
 (segment (start 96.52 49.022) (end 96.774 49.276) (width 1) (layer "B.Cu") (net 14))
 (segment (start 75.21 44.704) (end 74.93 44.984) (width 1) (layer "B.Cu") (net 14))
 (segment (start 58.326032 42.672) (end 59.770016 41.228016) (width 1) (layer "B.Cu") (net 14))
 (segment (start 62.23 56.388) (end 58.326032 52.484032) (width 0.5) (layer "B.Cu") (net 14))
 (segment (start 58.326032 52.484032) (end 58.326032 47.244) (width 0.5) (layer "B.Cu") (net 14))
 (segment (start 72.266 45.844) (end 72.771 45.339) (width 0.5) (layer "B.Cu") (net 14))
 (segment (start 75.21 54.838) (end 73.66 56.388) (width 0.5) (layer "B.Cu") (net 14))
 (segment (start 75.21 54.102) (end 75.21 53.568) (width 0.5) (layer "B.Cu") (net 14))
 (segment (start 91.694 44.704) (end 91.44 44.704) (width 1) (layer "B.Cu") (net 14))
 (segment (start 58.326032 47.244) (end 63.5 47.244) (width 0.5) (layer "B.Cu") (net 14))
 (segment (start 52.832 39.878) (end 55.626 42.672) (width 1) (layer "B.Cu") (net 14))
 (segment (start 73.152 44.958) (end 73.178 44.984) (width 0.5) (layer "B.Cu") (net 14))
 (segment (start 91.44 44.704) (end 89.154 46.99) (width 1) (layer "B.Cu") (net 14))
 (segment (start 95.423984 29.036016) (end 100.249984 29.036016) (width 1) (layer "B.Cu") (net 14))
 (segment (start 100.249984 29.036016) (end 100.503984 29.036016) (width 1) (layer "B.Cu") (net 14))
 (segment (start 67.574979 24.13) (end 68.596187 25.151208) (width 0.5) (layer "B.Cu") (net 13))
 (segment (start 101.854 52.578) (end 95.25 59.182) (width 0.5) (layer "B.Cu") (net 13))
 (segment (start 51.308 51.562) (end 51.308 33.274) (width 0.5) (layer "B.Cu") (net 13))
 (segment (start 58.928 59.182) (end 51.308 51.562) (width 0.5) (layer "B.Cu") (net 13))
 (segment (start 60.452 24.13) (end 67.574979 24.13) (width 0.5) (layer "B.Cu") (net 13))
 (segment (start 101.854 49.276) (end 101.854 52.578) (width 0.5) (layer "B.Cu") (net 13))
 (segment (start 95.25 59.182) (end 58.928 59.182) (width 0.5) (layer "B.Cu") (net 13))
 (segment (start 51.308 33.274) (end 60.452 24.13) (width 0.5) (layer "B.Cu") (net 13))
 (segment (start 107.732102 28.720051) (end 112.032051 28.720051) (width 0.5) (layer "B.Cu") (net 11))
 (segment (start 112.032051 28.720051) (end 119.888 36.576) (width 0.5) (layer "B.Cu") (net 11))
 (segment (start 119.888 36.576) (end 119.888 38.354) (width 0.5) (layer "B.Cu") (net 11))
 (segment (start 119.888 38.354) (end 108.966 49.276) (width 0.5) (layer "B.Cu") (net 11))
 (segment (start 108.966 49.276) (end 106.934 49.276) (width 0.5) (layer "B.Cu") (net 11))
 (segment (start 97.028 41.91) (end 88.392 41.91) (width 0.5) (layer "F.Cu") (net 12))
 (segment (start 88.392 41.91) (end 85.598 39.116) (width 0.5) (layer "F.Cu") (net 12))
 (via (at 85.598 39.116) (size 1.8) (drill 1) (layers "F.Cu" "B.Cu") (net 12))
 (via (at 97.028 41.91) (size 1.8) (drill 1) (layers "F.Cu" "B.Cu") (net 12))
 (segment (start 82.442 39.116) (end 82.042 39.516) (width 0.5) (layer "B.Cu") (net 12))
 (segment (start 97.282 42.164) (end 97.028 41.91) (width 0.5) (layer "B.Cu") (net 12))
 (segment (start 103.886 42.164) (end 97.282 42.164) (width 0.5) (layer "B.Cu") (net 12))
 (segment (start 85.598 39.116) (end 82.442 39.116) (width 0.5) (layer "B.Cu") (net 12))
 (segment (start 104.394 49.276) (end 104.394 42.672) (width 0.5) (layer "B.Cu") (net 12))
 (segment (start 104.394 42.672) (end 103.886 42.164) (width 0.5) (layer "B.Cu") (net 12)))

